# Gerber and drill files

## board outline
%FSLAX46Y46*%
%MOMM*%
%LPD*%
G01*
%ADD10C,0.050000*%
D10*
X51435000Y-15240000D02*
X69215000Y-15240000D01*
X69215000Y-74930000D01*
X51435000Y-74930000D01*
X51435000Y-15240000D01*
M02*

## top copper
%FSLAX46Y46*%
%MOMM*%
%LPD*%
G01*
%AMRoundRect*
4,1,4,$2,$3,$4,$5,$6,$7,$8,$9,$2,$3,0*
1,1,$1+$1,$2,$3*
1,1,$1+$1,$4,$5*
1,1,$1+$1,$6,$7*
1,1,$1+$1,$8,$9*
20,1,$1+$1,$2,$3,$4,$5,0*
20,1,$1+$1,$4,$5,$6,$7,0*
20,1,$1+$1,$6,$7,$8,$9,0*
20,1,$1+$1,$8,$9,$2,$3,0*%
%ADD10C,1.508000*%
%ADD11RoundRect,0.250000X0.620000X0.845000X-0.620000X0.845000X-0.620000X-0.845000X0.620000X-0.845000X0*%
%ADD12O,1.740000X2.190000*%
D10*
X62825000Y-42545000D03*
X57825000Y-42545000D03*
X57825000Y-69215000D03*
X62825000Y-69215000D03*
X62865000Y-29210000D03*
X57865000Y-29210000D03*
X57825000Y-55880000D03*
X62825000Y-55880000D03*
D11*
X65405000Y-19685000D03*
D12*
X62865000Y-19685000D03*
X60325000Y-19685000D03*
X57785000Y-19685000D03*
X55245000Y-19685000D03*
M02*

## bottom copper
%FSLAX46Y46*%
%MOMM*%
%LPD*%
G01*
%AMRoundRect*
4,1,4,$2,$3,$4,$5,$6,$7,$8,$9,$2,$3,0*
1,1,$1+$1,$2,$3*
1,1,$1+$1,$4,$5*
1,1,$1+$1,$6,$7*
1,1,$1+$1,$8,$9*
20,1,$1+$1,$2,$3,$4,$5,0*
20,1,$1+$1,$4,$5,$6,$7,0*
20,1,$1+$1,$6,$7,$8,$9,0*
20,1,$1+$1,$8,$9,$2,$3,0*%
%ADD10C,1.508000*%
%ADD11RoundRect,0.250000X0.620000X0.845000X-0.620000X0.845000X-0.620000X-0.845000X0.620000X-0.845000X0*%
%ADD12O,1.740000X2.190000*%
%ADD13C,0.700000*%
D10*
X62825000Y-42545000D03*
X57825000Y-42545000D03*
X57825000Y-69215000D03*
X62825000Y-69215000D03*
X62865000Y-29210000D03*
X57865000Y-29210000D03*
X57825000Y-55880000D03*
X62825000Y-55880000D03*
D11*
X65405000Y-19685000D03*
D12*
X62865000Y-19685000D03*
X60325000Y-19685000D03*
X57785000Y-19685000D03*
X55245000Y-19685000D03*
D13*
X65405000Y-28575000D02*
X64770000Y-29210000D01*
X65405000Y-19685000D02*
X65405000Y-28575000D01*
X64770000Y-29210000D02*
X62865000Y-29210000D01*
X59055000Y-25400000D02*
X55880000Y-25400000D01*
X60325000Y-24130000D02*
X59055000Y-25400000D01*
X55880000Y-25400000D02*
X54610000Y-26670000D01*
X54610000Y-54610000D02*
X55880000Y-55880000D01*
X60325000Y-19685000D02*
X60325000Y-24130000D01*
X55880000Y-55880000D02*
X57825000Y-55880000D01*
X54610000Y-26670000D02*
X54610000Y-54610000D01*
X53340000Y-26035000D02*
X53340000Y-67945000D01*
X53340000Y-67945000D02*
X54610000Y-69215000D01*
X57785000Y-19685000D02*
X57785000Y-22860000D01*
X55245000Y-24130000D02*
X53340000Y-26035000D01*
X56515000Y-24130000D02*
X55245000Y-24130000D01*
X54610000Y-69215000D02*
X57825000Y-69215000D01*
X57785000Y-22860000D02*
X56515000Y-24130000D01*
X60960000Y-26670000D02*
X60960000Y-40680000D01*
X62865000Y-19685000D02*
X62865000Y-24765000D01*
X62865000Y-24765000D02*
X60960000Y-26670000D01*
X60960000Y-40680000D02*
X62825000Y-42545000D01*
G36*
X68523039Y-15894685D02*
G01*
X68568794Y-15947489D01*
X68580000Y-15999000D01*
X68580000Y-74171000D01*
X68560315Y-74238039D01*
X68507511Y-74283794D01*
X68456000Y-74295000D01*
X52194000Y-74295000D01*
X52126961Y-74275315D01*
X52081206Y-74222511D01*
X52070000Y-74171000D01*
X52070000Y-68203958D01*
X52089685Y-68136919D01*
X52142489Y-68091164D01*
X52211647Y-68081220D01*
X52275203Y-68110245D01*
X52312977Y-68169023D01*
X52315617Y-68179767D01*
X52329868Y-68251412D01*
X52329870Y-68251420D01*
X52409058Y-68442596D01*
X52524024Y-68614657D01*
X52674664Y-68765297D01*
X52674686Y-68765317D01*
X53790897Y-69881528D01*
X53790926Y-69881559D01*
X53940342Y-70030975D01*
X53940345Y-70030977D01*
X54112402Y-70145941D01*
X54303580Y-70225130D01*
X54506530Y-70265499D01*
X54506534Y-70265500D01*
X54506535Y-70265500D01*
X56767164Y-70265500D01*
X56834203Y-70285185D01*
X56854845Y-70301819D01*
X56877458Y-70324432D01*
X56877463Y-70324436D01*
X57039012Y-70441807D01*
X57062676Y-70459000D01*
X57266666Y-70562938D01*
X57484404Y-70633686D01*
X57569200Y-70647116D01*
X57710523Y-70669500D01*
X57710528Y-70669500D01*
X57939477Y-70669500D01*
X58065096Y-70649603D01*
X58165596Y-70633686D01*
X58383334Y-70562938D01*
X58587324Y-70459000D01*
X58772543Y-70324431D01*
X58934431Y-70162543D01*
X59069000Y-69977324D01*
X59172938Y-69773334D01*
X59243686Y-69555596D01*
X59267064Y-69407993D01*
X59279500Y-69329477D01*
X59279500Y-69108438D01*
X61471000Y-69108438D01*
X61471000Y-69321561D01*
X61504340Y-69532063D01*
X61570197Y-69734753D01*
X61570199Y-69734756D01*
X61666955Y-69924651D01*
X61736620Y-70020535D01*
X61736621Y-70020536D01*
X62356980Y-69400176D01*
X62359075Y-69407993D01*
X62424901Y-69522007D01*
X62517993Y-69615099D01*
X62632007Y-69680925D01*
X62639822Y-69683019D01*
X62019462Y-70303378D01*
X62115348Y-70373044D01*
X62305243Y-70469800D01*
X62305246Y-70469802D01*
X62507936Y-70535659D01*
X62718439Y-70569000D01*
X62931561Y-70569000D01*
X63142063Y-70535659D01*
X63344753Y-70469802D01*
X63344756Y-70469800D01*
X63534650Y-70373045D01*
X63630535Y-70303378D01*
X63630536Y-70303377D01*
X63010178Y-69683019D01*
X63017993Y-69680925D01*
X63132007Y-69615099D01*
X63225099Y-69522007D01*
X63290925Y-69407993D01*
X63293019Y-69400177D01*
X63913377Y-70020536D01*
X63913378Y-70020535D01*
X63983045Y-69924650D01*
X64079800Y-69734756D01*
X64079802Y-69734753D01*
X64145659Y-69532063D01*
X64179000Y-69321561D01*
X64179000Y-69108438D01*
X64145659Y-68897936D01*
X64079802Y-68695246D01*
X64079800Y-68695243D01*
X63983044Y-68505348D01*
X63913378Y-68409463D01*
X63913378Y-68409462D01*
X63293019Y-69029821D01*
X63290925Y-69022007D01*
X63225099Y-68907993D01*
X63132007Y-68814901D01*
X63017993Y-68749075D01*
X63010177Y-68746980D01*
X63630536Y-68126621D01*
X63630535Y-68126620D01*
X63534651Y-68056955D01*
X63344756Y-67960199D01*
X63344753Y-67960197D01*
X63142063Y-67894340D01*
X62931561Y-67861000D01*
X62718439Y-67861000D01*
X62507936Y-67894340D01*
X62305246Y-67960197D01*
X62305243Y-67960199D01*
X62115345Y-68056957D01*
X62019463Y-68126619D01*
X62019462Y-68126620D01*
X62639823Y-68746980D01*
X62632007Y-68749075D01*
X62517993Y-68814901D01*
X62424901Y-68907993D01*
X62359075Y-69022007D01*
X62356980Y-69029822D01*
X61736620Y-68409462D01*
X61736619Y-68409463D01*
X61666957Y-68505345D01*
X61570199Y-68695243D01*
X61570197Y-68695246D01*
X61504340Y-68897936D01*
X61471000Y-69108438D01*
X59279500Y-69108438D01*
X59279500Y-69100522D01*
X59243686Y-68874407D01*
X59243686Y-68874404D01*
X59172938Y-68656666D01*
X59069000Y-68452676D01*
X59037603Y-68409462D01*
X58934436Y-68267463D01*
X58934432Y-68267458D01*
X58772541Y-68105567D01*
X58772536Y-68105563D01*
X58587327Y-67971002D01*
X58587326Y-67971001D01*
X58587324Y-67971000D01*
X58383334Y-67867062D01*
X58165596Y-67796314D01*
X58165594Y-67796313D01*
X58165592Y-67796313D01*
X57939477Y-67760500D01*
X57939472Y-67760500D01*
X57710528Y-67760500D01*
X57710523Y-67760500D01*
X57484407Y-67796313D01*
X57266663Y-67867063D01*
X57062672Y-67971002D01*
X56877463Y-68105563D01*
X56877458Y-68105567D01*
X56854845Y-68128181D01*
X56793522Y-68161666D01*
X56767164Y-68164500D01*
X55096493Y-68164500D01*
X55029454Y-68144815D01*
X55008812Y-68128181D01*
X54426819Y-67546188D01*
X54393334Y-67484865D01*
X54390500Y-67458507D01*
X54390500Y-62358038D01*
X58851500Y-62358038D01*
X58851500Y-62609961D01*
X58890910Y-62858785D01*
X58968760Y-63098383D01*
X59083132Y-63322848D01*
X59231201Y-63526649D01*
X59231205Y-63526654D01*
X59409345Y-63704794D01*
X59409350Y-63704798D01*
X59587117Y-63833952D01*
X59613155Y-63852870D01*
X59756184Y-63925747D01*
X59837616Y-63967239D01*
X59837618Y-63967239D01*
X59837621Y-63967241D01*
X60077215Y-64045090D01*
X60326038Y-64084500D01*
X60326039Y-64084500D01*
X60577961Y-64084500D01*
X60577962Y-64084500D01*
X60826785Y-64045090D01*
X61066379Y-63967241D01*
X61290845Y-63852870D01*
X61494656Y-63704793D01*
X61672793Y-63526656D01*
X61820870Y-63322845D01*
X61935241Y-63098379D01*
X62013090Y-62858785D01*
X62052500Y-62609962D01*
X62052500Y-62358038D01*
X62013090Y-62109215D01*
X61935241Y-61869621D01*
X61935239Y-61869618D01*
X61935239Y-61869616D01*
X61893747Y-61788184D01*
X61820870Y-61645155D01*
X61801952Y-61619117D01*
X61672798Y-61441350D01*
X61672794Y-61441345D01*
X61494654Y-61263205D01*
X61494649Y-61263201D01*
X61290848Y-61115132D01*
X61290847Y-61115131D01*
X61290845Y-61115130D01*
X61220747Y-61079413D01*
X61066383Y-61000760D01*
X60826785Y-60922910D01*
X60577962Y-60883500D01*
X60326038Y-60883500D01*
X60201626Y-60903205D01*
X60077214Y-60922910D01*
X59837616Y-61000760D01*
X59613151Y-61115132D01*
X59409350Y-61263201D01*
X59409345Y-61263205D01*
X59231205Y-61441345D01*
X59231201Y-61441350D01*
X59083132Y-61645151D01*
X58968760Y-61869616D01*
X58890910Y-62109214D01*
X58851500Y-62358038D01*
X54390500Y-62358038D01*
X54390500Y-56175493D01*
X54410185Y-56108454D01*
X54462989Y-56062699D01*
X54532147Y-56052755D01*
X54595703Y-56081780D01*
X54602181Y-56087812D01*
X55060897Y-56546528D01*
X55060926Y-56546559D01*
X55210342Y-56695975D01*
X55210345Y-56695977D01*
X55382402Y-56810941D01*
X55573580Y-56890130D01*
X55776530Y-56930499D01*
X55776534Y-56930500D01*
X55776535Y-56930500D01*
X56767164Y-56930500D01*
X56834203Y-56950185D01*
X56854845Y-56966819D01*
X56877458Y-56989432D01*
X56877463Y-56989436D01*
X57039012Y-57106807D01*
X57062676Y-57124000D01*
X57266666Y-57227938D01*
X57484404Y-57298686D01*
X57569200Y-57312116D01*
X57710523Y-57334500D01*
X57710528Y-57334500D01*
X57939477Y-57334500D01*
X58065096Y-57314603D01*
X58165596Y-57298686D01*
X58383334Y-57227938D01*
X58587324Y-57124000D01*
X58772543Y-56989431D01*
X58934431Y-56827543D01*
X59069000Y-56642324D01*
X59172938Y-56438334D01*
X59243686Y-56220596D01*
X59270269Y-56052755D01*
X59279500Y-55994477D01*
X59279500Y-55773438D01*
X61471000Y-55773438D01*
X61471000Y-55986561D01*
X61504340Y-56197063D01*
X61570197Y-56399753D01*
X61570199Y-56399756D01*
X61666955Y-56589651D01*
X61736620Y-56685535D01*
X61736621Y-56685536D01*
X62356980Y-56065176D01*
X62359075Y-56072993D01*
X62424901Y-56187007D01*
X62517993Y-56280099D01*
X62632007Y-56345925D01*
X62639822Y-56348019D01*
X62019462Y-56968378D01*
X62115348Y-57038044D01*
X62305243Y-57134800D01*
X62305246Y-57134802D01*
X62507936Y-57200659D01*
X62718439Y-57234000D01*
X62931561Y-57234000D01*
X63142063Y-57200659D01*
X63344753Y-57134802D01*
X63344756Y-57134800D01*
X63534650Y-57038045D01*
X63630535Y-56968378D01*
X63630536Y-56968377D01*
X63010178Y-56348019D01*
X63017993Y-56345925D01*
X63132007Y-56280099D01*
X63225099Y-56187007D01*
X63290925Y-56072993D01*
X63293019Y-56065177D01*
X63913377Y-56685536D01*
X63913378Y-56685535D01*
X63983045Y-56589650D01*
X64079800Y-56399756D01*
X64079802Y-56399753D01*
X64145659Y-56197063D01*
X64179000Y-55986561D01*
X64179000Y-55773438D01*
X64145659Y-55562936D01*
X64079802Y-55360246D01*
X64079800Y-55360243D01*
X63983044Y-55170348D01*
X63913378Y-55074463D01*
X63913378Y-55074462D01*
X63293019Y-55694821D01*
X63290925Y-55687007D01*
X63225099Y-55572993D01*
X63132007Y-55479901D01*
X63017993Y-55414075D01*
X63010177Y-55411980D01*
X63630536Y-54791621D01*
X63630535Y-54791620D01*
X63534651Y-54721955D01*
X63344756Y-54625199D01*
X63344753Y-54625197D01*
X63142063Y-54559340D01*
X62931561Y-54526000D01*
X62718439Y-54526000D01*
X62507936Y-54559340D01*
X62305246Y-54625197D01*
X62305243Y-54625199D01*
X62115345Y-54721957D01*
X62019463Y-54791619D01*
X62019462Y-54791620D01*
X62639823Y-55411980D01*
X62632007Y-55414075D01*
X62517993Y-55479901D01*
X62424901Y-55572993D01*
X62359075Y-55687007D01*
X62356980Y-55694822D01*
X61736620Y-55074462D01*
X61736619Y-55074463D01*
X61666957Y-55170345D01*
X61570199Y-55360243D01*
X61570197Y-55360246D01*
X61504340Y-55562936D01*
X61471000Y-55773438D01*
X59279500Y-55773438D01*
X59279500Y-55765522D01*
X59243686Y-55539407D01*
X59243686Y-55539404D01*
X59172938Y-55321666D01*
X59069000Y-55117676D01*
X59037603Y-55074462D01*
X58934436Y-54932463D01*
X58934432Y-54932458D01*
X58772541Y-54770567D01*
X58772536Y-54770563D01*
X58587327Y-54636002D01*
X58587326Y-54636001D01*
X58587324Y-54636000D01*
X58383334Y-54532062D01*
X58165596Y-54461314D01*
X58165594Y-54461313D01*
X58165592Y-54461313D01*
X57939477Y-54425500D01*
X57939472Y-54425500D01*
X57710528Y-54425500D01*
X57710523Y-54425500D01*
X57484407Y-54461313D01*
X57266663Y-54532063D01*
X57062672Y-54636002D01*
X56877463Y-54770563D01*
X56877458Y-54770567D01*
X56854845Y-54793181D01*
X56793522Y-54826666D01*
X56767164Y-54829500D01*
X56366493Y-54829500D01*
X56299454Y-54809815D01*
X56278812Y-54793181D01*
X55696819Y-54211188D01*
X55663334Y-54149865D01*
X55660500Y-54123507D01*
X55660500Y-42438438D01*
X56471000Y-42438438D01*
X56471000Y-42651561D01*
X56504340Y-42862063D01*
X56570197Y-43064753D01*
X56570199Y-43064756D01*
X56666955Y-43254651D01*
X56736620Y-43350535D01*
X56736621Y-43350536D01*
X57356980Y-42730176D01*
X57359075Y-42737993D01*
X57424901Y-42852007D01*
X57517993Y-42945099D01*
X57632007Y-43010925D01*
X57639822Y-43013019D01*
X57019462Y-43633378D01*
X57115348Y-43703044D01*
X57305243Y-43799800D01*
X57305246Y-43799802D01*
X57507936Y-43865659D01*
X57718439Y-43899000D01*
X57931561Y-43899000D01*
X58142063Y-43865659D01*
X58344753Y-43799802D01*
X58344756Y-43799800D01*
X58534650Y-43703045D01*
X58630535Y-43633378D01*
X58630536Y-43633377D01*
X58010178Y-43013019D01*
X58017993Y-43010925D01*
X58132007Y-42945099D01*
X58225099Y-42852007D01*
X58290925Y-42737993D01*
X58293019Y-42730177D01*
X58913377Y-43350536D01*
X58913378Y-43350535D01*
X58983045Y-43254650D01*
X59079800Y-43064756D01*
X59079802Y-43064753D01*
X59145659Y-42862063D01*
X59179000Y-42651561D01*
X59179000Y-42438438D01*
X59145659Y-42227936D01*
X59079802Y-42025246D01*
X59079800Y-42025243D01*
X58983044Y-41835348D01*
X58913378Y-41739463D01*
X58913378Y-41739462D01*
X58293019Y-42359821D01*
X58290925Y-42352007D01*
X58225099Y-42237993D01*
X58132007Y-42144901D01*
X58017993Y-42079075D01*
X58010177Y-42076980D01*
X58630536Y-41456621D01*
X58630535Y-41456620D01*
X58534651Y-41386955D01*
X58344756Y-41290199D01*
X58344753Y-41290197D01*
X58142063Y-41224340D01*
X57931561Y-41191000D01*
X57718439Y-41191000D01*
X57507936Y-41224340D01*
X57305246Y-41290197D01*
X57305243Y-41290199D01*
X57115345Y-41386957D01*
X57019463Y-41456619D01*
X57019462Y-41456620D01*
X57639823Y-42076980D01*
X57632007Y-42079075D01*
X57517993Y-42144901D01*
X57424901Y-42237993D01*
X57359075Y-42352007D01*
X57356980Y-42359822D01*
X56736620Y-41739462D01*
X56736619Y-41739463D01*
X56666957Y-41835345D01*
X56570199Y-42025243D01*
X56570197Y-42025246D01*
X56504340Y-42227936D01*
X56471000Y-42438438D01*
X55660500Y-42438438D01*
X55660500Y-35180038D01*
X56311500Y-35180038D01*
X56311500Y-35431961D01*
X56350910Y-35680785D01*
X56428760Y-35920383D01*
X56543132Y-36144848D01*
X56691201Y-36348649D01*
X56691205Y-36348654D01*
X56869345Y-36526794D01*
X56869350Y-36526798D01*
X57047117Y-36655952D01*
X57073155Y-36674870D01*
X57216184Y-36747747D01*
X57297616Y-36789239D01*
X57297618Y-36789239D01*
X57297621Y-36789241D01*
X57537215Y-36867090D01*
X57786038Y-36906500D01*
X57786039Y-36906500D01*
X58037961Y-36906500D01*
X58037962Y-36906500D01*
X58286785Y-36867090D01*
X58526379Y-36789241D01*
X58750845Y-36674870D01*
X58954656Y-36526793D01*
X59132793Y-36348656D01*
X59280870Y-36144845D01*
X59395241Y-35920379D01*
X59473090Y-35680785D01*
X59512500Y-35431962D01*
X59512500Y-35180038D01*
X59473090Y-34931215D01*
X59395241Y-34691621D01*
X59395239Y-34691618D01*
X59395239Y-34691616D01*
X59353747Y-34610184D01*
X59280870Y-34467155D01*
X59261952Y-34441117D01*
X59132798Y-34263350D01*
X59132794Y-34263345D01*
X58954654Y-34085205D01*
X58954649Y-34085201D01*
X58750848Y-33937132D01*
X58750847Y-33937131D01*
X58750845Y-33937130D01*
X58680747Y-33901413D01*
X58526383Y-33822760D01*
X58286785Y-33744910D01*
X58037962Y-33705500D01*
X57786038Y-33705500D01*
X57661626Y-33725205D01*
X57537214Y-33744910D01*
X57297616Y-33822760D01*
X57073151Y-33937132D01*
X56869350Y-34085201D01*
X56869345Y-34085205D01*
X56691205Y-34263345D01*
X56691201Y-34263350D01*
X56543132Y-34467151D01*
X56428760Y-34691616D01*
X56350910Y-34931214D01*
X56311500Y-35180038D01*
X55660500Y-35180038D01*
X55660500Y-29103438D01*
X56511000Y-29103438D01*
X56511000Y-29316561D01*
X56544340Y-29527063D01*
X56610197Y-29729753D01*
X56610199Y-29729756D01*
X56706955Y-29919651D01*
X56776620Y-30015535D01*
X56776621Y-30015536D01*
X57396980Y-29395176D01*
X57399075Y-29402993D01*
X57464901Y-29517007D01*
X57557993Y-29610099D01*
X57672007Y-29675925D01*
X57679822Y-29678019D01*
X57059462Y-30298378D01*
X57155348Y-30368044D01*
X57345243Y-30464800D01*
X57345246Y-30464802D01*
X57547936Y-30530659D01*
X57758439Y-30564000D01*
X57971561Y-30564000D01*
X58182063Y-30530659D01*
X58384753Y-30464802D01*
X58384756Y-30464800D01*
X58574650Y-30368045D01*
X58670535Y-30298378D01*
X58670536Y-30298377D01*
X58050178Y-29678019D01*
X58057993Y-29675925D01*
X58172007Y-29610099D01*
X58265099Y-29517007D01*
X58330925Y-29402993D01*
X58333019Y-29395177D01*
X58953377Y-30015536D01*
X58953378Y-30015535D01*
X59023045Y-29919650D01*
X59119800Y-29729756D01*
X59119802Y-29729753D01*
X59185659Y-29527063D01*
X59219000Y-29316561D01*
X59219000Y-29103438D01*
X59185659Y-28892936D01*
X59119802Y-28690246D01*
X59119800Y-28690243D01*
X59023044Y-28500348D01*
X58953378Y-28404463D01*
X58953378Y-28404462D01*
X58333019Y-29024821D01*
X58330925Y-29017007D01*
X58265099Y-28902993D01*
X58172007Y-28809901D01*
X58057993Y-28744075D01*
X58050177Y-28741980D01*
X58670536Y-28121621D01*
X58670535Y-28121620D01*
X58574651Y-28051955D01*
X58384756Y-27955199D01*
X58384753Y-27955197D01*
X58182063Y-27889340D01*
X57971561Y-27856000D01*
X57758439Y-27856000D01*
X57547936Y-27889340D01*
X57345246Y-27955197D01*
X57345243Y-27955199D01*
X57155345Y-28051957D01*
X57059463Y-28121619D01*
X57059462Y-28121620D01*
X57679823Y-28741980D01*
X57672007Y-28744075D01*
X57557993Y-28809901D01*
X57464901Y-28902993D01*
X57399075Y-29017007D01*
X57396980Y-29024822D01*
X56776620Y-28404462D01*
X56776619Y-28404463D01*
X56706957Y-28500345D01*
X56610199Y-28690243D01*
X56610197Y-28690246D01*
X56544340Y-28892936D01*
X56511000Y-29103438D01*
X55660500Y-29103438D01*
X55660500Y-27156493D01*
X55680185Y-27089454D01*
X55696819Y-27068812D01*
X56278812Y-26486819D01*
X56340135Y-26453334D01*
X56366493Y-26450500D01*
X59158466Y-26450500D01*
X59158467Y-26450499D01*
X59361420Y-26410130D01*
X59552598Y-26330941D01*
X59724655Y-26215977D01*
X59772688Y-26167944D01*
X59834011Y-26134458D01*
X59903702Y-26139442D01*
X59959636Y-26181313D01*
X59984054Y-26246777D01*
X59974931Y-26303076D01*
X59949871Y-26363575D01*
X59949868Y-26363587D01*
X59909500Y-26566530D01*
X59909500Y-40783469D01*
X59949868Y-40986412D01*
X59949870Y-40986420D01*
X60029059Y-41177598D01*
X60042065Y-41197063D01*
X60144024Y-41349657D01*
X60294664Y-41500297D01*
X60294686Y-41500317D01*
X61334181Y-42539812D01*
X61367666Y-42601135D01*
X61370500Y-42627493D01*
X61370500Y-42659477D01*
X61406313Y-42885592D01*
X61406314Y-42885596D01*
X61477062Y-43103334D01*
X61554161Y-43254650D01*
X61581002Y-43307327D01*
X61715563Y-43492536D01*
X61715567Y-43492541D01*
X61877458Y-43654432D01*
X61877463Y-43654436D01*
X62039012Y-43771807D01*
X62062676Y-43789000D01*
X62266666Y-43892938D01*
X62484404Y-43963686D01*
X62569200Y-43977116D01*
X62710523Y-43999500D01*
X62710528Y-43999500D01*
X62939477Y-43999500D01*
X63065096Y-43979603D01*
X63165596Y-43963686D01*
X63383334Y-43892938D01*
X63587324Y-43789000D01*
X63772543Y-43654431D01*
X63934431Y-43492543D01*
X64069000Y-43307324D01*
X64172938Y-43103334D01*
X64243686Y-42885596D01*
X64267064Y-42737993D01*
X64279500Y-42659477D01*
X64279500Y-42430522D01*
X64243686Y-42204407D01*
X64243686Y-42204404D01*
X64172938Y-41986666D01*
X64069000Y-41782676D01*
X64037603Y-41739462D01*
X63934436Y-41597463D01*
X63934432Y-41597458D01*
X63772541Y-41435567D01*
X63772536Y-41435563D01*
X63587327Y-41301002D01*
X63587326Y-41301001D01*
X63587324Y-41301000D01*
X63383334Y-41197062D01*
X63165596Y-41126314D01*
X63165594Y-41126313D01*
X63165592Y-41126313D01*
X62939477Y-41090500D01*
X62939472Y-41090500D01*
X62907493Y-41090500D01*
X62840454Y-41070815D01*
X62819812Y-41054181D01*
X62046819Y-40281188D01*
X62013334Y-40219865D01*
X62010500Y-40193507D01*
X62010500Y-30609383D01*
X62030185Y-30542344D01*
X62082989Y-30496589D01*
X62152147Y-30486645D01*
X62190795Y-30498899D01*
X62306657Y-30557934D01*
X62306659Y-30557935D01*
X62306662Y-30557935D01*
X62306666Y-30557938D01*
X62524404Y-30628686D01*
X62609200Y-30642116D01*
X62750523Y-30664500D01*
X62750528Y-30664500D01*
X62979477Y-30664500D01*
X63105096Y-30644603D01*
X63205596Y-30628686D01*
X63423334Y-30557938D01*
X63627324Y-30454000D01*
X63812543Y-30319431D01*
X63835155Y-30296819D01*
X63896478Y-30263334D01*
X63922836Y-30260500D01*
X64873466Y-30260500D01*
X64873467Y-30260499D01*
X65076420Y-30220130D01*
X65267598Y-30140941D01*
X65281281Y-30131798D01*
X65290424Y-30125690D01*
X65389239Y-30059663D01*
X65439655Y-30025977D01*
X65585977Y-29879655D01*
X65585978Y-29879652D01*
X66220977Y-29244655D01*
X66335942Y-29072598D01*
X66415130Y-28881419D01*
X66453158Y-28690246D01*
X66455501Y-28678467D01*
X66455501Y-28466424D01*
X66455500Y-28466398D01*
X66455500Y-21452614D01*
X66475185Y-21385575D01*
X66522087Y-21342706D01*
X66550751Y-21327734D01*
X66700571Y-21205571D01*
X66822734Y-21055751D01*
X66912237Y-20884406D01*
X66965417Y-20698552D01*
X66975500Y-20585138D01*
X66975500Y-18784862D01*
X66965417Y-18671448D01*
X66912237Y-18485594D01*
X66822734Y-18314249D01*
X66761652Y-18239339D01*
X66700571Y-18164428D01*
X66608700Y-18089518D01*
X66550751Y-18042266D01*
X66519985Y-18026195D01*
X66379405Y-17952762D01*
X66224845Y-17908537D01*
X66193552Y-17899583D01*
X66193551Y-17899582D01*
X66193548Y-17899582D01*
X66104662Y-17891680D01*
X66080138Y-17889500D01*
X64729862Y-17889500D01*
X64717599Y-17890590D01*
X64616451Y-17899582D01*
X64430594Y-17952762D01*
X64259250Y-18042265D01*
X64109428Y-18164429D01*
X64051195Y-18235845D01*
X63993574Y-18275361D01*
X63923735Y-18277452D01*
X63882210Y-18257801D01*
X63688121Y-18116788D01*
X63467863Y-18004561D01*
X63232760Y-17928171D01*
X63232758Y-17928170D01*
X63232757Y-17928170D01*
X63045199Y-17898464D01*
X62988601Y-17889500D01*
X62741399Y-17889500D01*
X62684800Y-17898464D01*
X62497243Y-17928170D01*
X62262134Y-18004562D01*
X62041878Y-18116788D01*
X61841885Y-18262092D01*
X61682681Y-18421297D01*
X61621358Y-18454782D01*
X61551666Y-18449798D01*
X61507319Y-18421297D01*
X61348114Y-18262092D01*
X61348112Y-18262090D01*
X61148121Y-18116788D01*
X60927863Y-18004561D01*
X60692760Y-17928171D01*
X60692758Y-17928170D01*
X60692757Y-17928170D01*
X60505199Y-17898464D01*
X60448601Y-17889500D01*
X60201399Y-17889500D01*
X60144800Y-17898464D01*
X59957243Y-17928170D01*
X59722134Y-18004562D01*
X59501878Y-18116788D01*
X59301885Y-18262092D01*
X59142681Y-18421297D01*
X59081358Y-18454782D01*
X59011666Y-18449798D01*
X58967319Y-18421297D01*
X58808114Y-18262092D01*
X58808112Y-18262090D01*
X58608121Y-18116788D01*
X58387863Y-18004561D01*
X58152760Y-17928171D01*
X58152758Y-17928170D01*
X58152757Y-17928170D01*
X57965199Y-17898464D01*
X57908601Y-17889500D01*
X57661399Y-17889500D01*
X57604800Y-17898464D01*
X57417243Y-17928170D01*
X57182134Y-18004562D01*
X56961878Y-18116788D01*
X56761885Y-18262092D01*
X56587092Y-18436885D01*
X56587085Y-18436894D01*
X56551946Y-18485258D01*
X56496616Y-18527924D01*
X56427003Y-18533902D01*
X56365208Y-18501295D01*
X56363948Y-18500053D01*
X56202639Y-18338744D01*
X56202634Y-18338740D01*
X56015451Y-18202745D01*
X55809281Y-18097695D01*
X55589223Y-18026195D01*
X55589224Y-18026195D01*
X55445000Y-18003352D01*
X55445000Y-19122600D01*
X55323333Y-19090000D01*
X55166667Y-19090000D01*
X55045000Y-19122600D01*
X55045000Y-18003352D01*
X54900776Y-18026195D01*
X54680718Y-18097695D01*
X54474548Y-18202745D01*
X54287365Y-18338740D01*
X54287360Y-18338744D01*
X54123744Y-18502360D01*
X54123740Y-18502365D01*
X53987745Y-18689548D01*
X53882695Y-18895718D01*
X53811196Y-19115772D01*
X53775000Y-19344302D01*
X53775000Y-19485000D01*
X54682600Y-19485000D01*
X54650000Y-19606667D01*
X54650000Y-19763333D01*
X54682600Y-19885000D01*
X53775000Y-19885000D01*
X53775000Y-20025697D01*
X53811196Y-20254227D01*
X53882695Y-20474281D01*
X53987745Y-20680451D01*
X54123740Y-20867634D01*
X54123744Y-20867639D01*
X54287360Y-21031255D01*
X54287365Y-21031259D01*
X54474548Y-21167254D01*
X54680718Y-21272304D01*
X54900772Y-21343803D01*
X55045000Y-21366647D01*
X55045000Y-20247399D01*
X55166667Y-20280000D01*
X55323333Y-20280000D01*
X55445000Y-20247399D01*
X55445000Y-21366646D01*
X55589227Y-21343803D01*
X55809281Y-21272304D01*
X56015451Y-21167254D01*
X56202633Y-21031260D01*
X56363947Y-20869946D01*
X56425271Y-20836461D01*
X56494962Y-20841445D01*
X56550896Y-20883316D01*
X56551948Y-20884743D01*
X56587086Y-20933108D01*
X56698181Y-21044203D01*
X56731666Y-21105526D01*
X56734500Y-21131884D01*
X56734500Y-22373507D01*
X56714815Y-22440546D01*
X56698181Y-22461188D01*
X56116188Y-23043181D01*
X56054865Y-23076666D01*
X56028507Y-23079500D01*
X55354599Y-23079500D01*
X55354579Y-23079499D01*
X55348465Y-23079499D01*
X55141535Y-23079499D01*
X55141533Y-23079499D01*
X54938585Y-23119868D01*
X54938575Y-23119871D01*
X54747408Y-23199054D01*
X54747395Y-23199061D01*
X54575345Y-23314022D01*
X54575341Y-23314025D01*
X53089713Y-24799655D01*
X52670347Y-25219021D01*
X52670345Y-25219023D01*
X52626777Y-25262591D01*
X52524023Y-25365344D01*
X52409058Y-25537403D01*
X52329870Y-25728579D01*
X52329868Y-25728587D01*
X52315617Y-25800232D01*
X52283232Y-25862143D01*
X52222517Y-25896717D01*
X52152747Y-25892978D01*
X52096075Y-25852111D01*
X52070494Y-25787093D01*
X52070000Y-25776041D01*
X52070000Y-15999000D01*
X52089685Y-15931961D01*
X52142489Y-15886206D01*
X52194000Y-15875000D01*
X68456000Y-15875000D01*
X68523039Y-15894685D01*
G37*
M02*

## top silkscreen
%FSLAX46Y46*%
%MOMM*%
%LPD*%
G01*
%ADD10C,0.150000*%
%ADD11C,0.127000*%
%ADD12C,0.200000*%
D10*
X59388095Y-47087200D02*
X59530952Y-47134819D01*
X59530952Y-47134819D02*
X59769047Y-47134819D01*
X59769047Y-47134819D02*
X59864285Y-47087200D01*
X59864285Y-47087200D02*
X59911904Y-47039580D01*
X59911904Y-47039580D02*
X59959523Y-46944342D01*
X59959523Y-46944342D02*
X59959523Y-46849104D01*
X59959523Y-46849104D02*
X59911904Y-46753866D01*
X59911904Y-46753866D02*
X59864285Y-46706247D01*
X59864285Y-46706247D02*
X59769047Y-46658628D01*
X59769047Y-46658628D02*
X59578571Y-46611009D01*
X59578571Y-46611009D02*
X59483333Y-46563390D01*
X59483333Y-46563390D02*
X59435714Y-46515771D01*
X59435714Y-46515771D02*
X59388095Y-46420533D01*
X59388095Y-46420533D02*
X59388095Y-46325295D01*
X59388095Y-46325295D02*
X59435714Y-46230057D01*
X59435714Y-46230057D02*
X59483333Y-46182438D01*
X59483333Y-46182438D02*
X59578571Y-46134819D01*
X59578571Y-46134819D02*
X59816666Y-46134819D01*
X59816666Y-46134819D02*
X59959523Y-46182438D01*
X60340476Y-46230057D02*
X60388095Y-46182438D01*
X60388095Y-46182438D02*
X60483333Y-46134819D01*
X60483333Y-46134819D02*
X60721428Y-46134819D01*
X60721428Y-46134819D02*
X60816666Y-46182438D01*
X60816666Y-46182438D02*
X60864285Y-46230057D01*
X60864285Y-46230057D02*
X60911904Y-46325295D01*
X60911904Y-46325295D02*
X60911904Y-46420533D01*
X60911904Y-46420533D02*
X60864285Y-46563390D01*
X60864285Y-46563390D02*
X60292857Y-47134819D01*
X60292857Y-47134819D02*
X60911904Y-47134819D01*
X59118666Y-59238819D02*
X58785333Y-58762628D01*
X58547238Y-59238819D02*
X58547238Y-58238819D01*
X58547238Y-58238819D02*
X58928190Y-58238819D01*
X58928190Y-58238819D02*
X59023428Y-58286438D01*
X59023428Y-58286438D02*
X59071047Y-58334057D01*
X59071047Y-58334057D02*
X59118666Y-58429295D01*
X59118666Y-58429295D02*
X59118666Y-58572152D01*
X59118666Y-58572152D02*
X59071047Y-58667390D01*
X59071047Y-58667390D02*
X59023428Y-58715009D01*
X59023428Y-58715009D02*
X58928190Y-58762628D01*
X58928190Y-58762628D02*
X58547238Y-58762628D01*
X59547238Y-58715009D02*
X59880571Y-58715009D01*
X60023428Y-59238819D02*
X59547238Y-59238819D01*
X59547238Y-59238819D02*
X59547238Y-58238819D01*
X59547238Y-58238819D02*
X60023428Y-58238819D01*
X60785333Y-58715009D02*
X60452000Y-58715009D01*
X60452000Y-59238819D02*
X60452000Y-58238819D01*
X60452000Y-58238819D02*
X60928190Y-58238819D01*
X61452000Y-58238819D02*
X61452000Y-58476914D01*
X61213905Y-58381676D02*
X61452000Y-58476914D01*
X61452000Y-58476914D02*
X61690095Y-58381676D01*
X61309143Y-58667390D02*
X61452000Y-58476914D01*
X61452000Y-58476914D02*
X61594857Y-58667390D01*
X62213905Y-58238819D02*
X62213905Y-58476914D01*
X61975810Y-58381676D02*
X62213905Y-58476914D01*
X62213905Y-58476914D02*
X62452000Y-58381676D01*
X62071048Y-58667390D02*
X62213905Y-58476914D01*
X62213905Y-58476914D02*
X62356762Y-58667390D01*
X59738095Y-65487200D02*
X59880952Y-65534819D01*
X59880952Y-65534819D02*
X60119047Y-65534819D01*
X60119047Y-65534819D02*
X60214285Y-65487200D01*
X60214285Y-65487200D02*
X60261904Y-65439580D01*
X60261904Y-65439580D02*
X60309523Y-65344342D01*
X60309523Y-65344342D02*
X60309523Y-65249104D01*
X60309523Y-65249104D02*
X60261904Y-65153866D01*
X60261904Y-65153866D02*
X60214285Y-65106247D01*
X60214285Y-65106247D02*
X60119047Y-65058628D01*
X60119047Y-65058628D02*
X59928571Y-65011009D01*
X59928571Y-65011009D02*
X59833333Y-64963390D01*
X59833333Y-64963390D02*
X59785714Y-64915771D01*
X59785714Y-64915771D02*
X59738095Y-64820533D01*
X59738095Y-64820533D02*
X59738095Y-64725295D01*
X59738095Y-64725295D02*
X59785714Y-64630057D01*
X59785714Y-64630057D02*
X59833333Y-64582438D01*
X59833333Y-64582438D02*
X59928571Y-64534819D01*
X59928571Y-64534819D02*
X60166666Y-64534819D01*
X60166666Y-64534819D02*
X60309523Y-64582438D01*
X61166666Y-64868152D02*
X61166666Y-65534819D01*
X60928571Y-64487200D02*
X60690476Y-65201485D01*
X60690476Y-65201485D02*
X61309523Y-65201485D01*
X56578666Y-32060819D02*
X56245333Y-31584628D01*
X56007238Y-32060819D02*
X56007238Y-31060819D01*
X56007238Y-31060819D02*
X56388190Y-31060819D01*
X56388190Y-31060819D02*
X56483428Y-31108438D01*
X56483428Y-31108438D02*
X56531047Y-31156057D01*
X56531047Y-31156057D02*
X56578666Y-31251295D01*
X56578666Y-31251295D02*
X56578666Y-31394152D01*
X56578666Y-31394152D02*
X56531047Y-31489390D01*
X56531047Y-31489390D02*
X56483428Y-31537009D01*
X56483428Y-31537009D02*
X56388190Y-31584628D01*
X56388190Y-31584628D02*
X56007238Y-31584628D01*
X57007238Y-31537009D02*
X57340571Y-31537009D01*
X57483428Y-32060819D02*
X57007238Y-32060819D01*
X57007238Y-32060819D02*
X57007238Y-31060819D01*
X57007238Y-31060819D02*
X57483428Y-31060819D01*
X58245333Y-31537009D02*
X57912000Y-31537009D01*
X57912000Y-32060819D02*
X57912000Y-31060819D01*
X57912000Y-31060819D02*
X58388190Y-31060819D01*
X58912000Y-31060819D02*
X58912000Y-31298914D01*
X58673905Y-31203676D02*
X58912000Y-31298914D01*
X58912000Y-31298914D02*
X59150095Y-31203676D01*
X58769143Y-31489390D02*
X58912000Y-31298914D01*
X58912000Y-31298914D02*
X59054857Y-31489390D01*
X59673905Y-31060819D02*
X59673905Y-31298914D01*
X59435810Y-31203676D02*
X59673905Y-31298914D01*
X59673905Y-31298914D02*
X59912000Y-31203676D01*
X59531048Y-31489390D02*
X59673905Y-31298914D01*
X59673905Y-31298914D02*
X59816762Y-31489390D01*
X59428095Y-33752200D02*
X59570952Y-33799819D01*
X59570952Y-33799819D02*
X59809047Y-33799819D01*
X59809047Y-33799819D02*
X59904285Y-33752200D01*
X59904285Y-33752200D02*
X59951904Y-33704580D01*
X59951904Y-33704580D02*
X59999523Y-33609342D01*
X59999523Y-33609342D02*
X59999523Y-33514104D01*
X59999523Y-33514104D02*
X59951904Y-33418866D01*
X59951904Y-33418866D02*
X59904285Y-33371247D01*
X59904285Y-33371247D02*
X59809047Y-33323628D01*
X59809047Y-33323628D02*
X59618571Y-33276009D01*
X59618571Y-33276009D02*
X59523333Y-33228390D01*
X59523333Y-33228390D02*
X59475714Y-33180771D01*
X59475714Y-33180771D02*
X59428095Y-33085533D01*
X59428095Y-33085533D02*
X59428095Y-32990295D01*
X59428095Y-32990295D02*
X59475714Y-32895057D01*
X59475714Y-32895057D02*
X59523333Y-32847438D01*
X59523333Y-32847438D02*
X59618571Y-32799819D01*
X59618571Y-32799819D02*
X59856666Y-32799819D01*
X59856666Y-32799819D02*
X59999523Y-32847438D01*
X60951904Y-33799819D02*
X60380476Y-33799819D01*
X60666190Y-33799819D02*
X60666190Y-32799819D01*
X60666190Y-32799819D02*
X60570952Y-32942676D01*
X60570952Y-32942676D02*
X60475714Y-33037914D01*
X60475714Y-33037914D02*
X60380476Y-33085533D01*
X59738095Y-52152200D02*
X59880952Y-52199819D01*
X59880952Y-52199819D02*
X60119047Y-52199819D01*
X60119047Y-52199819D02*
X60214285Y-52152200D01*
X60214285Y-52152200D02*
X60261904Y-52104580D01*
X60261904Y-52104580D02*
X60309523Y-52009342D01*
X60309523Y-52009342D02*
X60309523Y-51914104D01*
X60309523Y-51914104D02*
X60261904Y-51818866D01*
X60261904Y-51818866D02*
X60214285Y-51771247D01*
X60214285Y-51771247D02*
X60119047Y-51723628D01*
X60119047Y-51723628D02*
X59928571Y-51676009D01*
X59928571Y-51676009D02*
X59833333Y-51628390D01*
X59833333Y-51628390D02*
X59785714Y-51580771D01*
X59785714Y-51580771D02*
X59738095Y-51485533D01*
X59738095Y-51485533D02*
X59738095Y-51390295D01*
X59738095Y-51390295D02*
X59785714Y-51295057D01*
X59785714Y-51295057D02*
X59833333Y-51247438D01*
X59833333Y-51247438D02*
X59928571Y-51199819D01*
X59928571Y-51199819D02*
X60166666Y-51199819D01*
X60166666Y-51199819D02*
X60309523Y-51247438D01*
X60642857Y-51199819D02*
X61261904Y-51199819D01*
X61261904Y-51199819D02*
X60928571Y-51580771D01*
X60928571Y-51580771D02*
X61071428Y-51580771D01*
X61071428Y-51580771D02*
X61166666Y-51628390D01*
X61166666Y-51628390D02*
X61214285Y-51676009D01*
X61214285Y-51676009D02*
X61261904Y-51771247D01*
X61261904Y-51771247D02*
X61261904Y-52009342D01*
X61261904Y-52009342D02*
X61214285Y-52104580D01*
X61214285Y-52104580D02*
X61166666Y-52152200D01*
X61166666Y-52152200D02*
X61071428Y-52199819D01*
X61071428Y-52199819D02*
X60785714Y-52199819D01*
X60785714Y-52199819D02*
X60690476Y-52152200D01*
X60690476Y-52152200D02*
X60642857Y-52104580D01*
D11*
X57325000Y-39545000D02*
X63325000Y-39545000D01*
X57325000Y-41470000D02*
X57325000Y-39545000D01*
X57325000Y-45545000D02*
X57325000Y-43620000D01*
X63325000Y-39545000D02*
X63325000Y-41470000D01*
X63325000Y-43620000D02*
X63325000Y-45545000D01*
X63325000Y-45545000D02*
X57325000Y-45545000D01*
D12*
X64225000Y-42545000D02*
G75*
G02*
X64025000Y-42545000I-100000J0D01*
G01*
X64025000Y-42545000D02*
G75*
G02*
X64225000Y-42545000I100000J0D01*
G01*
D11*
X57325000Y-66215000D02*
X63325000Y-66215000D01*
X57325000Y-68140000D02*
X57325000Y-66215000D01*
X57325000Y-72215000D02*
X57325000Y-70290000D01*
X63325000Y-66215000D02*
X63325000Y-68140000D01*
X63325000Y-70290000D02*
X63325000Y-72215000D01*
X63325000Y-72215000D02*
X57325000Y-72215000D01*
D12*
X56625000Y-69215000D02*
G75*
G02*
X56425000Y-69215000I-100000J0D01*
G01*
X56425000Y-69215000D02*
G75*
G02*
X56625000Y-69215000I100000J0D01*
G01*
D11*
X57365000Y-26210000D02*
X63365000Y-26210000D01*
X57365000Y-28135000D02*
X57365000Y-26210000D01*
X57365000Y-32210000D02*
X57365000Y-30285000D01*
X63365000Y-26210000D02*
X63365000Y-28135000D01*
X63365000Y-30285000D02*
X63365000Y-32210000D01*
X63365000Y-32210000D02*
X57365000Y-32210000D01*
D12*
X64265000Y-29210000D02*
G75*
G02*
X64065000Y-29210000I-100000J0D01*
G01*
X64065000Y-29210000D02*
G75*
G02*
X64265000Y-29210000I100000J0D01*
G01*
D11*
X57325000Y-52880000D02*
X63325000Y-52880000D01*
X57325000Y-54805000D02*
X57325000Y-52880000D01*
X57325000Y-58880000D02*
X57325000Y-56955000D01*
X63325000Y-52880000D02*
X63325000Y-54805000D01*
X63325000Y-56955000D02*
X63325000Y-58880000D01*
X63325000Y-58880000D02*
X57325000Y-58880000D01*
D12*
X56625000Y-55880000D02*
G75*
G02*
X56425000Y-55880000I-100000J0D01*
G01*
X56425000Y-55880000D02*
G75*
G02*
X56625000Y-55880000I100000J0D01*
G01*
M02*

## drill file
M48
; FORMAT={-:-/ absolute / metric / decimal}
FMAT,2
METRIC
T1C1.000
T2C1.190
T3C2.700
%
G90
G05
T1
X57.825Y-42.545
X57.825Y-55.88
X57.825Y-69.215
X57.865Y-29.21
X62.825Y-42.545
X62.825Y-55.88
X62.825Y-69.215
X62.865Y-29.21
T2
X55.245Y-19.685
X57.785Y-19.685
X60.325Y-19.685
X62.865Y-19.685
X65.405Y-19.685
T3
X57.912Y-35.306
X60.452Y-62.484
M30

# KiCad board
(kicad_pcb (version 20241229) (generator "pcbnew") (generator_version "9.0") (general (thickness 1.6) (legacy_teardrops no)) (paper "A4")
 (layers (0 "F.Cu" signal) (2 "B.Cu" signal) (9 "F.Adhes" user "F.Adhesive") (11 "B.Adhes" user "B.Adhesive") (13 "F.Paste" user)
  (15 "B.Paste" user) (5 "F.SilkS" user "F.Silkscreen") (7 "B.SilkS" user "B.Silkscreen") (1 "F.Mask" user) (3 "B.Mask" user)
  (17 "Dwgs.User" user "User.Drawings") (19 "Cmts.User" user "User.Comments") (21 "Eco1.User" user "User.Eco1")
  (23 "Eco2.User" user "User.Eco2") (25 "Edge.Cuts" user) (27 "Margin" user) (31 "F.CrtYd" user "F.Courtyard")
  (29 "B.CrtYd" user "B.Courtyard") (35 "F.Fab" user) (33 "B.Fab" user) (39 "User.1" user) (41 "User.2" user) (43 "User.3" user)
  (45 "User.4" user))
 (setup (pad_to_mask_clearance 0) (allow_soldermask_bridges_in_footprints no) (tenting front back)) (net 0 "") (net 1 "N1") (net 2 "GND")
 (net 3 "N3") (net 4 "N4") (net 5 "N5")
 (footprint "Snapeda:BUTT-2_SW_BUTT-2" (layer "F.Cu") (at 60.325 42.545 180)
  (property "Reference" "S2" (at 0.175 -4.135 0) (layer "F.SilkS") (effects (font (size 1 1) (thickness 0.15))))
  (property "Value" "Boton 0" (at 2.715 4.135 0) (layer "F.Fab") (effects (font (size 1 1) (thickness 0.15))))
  (fp_line (start 3 3) (end -3 3) (stroke (width 0.127) (type solid)) (layer "F.SilkS"))
  (fp_line (start 3 1.075) (end 3 3) (stroke (width 0.127) (type solid)) (layer "F.SilkS"))
  (fp_line (start 3 -3) (end 3 -1.075) (stroke (width 0.127) (type solid)) (layer "F.SilkS"))
  (fp_line (start -3 3) (end -3 1.075) (stroke (width 0.127) (type solid)) (layer "F.SilkS"))
  (fp_line (start -3 -1.075) (end -3 -3) (stroke (width 0.127) (type solid)) (layer "F.SilkS"))
  (fp_line (start -3 -3) (end 3 -3) (stroke (width 0.127) (type solid)) (layer "F.SilkS"))
  (fp_circle (center -3.8 0) (end -3.7 0) (stroke (width 0.2) (type solid)) (fill no) (layer "F.SilkS"))
  (pad "1" thru_hole circle (at -2.5 0 180) (size 1.508 1.508) (drill 1) (layers "*.Cu" "*.Mask") (remove_unused_layers no) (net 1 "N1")
   (solder_mask_margin 0.102))
  (pad "2" thru_hole circle (at 2.5 0 180) (size 1.508 1.508) (drill 1) (layers "*.Cu" "*.Mask") (remove_unused_layers no) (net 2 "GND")
   (solder_mask_margin 0.102)))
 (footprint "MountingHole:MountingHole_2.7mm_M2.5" (layer "F.Cu") (at 60.452 62.484)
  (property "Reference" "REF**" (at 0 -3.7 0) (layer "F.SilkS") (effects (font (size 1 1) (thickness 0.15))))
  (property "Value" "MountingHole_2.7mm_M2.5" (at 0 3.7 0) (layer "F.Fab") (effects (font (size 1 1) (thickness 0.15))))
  (pad "" np_thru_hole circle (at 0 0) (size 2.7 2.7) (drill 2.7) (layers "*.Cu" "*.Mask")))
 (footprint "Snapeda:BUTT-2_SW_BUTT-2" (layer "F.Cu") (at 60.325 69.215)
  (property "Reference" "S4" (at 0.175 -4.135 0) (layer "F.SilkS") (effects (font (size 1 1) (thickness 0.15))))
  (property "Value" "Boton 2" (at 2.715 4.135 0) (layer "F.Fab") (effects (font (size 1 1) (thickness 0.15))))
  (fp_line (start -3 -3) (end 3 -3) (stroke (width 0.127) (type solid)) (layer "F.SilkS"))
  (fp_line (start -3 -1.075) (end -3 -3) (stroke (width 0.127) (type solid)) (layer "F.SilkS"))
  (fp_line (start -3 3) (end -3 1.075) (stroke (width 0.127) (type solid)) (layer "F.SilkS"))
  (fp_line (start 3 -3) (end 3 -1.075) (stroke (width 0.127) (type solid)) (layer "F.SilkS"))
  (fp_line (start 3 1.075) (end 3 3) (stroke (width 0.127) (type solid)) (layer "F.SilkS"))
  (fp_line (start 3 3) (end -3 3) (stroke (width 0.127) (type solid)) (layer "F.SilkS"))
  (fp_circle (center -3.8 0) (end -3.7 0) (stroke (width 0.2) (type solid)) (fill no) (layer "F.SilkS"))
  (pad "1" thru_hole circle (at -2.5 0) (size 1.508 1.508) (drill 1) (layers "*.Cu" "*.Mask") (remove_unused_layers no) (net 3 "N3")
   (solder_mask_margin 0.102))
  (pad "2" thru_hole circle (at 2.5 0) (size 1.508 1.508) (drill 1) (layers "*.Cu" "*.Mask") (remove_unused_layers no) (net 2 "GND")
   (solder_mask_margin 0.102)))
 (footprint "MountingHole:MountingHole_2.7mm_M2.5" (layer "F.Cu") (at 57.912 35.306)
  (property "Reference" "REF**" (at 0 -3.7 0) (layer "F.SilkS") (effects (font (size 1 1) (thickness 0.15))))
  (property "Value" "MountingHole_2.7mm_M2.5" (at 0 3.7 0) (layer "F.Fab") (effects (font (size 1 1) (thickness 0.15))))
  (pad "" np_thru_hole circle (at 0 0) (size 2.7 2.7) (drill 2.7) (layers "*.Cu" "*.Mask")))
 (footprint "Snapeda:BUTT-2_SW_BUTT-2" (layer "F.Cu") (at 60.365 29.21 180)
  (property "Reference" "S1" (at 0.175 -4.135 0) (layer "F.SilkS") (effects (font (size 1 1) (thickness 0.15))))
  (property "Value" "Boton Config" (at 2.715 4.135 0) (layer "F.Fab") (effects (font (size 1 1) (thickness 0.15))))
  (fp_line (start 3 3) (end -3 3) (stroke (width 0.127) (type solid)) (layer "F.SilkS"))
  (fp_line (start 3 1.075) (end 3 3) (stroke (width 0.127) (type solid)) (layer "F.SilkS"))
  (fp_line (start 3 -3) (end 3 -1.075) (stroke (width 0.127) (type solid)) (layer "F.SilkS"))
  (fp_line (start -3 3) (end -3 1.075) (stroke (width 0.127) (type solid)) (layer "F.SilkS"))
  (fp_line (start -3 -1.075) (end -3 -3) (stroke (width 0.127) (type solid)) (layer "F.SilkS"))
  (fp_line (start -3 -3) (end 3 -3) (stroke (width 0.127) (type solid)) (layer "F.SilkS"))
  (fp_circle (center -3.8 0) (end -3.7 0) (stroke (width 0.2) (type solid)) (fill no) (layer "F.SilkS"))
  (pad "1" thru_hole circle (at -2.5 0 180) (size 1.508 1.508) (drill 1) (layers "*.Cu" "*.Mask") (remove_unused_layers no) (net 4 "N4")
   (solder_mask_margin 0.102))
  (pad "2" thru_hole circle (at 2.5 0 180) (size 1.508 1.508) (drill 1) (layers "*.Cu" "*.Mask") (remove_unused_layers no) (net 2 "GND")
   (solder_mask_margin 0.102)))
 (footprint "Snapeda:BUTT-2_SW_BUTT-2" (layer "F.Cu") (at 60.325 55.88)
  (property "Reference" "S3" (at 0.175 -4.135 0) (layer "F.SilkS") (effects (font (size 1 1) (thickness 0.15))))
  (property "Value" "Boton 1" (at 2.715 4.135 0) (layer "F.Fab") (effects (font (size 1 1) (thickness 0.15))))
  (fp_line (start -3 -3) (end 3 -3) (stroke (width 0.127) (type solid)) (layer "F.SilkS"))
  (fp_line (start -3 -1.075) (end -3 -3) (stroke (width 0.127) (type solid)) (layer "F.SilkS"))
  (fp_line (start -3 3) (end -3 1.075) (stroke (width 0.127) (type solid)) (layer "F.SilkS"))
  (fp_line (start 3 -3) (end 3 -1.075) (stroke (width 0.127) (type solid)) (layer "F.SilkS"))
  (fp_line (start 3 1.075) (end 3 3) (stroke (width 0.127) (type solid)) (layer "F.SilkS"))
  (fp_line (start 3 3) (end -3 3) (stroke (width 0.127) (type solid)) (layer "F.SilkS"))
  (fp_circle (center -3.8 0) (end -3.7 0) (stroke (width 0.2) (type solid)) (fill no) (layer "F.SilkS"))
  (pad "1" thru_hole circle (at -2.5 0) (size 1.508 1.508) (drill 1) (layers "*.Cu" "*.Mask") (remove_unused_layers no) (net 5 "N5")
   (solder_mask_margin 0.102))
  (pad "2" thru_hole circle (at 2.5 0) (size 1.508 1.508) (drill 1) (layers "*.Cu" "*.Mask") (remove_unused_layers no) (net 2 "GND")
   (solder_mask_margin 0.102)))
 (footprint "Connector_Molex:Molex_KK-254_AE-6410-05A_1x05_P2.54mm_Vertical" (layer "B.Cu") (at 65.405 19.685 180)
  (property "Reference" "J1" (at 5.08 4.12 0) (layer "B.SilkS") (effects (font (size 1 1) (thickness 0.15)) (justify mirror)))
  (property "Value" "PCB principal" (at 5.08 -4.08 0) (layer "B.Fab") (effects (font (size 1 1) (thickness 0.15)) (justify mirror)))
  (pad "1" thru_hole roundrect (at 0 0 180) (size 1.74 2.19) (drill 1.19) (layers "*.Cu" "*.Mask") (remove_unused_layers no)
   (roundrect_rratio 0.143678) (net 4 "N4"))
  (pad "2" thru_hole oval (at 2.54 0 180) (size 1.74 2.19) (drill 1.19) (layers "*.Cu" "*.Mask") (remove_unused_layers no) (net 1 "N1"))
  (pad "3" thru_hole oval (at 5.08 0 180) (size 1.74 2.19) (drill 1.19) (layers "*.Cu" "*.Mask") (remove_unused_layers no) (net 5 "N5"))
  (pad "4" thru_hole oval (at 7.62 0 180) (size 1.74 2.19) (drill 1.19) (layers "*.Cu" "*.Mask") (remove_unused_layers no) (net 3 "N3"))
  (pad "5" thru_hole oval (at 10.16 0 180) (size 1.74 2.19) (drill 1.19) (layers "*.Cu" "*.Mask") (remove_unused_layers no) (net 2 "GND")))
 (gr_rect (start 51.435 15.24) (end 69.215 74.93) (stroke (width 0.05) (type default)) (fill no) (layer "Edge.Cuts"))
 (segment (start 65.405 28.575) (end 64.77 29.21) (width 0.7) (layer "B.Cu") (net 4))
 (segment (start 65.405 19.685) (end 65.405 28.575) (width 0.7) (layer "B.Cu") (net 4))
 (segment (start 64.77 29.21) (end 62.865 29.21) (width 0.7) (layer "B.Cu") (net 4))
 (segment (start 59.055 25.4) (end 55.88 25.4) (width 0.7) (layer "B.Cu") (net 5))
 (segment (start 60.325 24.13) (end 59.055 25.4) (width 0.7) (layer "B.Cu") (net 5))
 (segment (start 55.88 25.4) (end 54.61 26.67) (width 0.7) (layer "B.Cu") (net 5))
 (segment (start 54.61 54.61) (end 55.88 55.88) (width 0.7) (layer "B.Cu") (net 5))
 (segment (start 60.325 19.685) (end 60.325 24.13) (width 0.7) (layer "B.Cu") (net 5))
 (segment (start 55.88 55.88) (end 57.825 55.88) (width 0.7) (layer "B.Cu") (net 5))
 (segment (start 54.61 26.67) (end 54.61 54.61) (width 0.7) (layer "B.Cu") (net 5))
 (segment (start 53.34 26.035) (end 53.34 67.945) (width 0.7) (layer "B.Cu") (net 3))
 (segment (start 53.34 67.945) (end 54.61 69.215) (width 0.7) (layer "B.Cu") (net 3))
 (segment (start 57.785 19.685) (end 57.785 22.86) (width 0.7) (layer "B.Cu") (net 3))
 (segment (start 55.245 24.13) (end 53.34 26.035) (width 0.7) (layer "B.Cu") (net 3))
 (segment (start 56.515 24.13) (end 55.245 24.13) (width 0.7) (layer "B.Cu") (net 3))
 (segment (start 54.61 69.215) (end 57.825 69.215) (width 0.7) (layer "B.Cu") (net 3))
 (segment (start 57.785 22.86) (end 56.515 24.13) (width 0.7) (layer "B.Cu") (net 3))
 (segment (start 60.96 26.67) (end 60.96 40.68) (width 0.7) (layer "B.Cu") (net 1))
 (segment (start 62.865 19.685) (end 62.865 24.765) (width 0.7) (layer "B.Cu") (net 1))
 (segment (start 62.865 24.765) (end 60.96 26.67) (width 0.7) (layer "B.Cu") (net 1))
 (segment (start 60.96 40.68) (end 62.825 42.545) (width 0.7) (layer "B.Cu") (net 1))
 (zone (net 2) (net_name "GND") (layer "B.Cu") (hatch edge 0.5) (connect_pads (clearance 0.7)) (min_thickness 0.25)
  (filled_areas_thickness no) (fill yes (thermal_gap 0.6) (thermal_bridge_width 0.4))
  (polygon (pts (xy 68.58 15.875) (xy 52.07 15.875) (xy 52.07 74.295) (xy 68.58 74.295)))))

